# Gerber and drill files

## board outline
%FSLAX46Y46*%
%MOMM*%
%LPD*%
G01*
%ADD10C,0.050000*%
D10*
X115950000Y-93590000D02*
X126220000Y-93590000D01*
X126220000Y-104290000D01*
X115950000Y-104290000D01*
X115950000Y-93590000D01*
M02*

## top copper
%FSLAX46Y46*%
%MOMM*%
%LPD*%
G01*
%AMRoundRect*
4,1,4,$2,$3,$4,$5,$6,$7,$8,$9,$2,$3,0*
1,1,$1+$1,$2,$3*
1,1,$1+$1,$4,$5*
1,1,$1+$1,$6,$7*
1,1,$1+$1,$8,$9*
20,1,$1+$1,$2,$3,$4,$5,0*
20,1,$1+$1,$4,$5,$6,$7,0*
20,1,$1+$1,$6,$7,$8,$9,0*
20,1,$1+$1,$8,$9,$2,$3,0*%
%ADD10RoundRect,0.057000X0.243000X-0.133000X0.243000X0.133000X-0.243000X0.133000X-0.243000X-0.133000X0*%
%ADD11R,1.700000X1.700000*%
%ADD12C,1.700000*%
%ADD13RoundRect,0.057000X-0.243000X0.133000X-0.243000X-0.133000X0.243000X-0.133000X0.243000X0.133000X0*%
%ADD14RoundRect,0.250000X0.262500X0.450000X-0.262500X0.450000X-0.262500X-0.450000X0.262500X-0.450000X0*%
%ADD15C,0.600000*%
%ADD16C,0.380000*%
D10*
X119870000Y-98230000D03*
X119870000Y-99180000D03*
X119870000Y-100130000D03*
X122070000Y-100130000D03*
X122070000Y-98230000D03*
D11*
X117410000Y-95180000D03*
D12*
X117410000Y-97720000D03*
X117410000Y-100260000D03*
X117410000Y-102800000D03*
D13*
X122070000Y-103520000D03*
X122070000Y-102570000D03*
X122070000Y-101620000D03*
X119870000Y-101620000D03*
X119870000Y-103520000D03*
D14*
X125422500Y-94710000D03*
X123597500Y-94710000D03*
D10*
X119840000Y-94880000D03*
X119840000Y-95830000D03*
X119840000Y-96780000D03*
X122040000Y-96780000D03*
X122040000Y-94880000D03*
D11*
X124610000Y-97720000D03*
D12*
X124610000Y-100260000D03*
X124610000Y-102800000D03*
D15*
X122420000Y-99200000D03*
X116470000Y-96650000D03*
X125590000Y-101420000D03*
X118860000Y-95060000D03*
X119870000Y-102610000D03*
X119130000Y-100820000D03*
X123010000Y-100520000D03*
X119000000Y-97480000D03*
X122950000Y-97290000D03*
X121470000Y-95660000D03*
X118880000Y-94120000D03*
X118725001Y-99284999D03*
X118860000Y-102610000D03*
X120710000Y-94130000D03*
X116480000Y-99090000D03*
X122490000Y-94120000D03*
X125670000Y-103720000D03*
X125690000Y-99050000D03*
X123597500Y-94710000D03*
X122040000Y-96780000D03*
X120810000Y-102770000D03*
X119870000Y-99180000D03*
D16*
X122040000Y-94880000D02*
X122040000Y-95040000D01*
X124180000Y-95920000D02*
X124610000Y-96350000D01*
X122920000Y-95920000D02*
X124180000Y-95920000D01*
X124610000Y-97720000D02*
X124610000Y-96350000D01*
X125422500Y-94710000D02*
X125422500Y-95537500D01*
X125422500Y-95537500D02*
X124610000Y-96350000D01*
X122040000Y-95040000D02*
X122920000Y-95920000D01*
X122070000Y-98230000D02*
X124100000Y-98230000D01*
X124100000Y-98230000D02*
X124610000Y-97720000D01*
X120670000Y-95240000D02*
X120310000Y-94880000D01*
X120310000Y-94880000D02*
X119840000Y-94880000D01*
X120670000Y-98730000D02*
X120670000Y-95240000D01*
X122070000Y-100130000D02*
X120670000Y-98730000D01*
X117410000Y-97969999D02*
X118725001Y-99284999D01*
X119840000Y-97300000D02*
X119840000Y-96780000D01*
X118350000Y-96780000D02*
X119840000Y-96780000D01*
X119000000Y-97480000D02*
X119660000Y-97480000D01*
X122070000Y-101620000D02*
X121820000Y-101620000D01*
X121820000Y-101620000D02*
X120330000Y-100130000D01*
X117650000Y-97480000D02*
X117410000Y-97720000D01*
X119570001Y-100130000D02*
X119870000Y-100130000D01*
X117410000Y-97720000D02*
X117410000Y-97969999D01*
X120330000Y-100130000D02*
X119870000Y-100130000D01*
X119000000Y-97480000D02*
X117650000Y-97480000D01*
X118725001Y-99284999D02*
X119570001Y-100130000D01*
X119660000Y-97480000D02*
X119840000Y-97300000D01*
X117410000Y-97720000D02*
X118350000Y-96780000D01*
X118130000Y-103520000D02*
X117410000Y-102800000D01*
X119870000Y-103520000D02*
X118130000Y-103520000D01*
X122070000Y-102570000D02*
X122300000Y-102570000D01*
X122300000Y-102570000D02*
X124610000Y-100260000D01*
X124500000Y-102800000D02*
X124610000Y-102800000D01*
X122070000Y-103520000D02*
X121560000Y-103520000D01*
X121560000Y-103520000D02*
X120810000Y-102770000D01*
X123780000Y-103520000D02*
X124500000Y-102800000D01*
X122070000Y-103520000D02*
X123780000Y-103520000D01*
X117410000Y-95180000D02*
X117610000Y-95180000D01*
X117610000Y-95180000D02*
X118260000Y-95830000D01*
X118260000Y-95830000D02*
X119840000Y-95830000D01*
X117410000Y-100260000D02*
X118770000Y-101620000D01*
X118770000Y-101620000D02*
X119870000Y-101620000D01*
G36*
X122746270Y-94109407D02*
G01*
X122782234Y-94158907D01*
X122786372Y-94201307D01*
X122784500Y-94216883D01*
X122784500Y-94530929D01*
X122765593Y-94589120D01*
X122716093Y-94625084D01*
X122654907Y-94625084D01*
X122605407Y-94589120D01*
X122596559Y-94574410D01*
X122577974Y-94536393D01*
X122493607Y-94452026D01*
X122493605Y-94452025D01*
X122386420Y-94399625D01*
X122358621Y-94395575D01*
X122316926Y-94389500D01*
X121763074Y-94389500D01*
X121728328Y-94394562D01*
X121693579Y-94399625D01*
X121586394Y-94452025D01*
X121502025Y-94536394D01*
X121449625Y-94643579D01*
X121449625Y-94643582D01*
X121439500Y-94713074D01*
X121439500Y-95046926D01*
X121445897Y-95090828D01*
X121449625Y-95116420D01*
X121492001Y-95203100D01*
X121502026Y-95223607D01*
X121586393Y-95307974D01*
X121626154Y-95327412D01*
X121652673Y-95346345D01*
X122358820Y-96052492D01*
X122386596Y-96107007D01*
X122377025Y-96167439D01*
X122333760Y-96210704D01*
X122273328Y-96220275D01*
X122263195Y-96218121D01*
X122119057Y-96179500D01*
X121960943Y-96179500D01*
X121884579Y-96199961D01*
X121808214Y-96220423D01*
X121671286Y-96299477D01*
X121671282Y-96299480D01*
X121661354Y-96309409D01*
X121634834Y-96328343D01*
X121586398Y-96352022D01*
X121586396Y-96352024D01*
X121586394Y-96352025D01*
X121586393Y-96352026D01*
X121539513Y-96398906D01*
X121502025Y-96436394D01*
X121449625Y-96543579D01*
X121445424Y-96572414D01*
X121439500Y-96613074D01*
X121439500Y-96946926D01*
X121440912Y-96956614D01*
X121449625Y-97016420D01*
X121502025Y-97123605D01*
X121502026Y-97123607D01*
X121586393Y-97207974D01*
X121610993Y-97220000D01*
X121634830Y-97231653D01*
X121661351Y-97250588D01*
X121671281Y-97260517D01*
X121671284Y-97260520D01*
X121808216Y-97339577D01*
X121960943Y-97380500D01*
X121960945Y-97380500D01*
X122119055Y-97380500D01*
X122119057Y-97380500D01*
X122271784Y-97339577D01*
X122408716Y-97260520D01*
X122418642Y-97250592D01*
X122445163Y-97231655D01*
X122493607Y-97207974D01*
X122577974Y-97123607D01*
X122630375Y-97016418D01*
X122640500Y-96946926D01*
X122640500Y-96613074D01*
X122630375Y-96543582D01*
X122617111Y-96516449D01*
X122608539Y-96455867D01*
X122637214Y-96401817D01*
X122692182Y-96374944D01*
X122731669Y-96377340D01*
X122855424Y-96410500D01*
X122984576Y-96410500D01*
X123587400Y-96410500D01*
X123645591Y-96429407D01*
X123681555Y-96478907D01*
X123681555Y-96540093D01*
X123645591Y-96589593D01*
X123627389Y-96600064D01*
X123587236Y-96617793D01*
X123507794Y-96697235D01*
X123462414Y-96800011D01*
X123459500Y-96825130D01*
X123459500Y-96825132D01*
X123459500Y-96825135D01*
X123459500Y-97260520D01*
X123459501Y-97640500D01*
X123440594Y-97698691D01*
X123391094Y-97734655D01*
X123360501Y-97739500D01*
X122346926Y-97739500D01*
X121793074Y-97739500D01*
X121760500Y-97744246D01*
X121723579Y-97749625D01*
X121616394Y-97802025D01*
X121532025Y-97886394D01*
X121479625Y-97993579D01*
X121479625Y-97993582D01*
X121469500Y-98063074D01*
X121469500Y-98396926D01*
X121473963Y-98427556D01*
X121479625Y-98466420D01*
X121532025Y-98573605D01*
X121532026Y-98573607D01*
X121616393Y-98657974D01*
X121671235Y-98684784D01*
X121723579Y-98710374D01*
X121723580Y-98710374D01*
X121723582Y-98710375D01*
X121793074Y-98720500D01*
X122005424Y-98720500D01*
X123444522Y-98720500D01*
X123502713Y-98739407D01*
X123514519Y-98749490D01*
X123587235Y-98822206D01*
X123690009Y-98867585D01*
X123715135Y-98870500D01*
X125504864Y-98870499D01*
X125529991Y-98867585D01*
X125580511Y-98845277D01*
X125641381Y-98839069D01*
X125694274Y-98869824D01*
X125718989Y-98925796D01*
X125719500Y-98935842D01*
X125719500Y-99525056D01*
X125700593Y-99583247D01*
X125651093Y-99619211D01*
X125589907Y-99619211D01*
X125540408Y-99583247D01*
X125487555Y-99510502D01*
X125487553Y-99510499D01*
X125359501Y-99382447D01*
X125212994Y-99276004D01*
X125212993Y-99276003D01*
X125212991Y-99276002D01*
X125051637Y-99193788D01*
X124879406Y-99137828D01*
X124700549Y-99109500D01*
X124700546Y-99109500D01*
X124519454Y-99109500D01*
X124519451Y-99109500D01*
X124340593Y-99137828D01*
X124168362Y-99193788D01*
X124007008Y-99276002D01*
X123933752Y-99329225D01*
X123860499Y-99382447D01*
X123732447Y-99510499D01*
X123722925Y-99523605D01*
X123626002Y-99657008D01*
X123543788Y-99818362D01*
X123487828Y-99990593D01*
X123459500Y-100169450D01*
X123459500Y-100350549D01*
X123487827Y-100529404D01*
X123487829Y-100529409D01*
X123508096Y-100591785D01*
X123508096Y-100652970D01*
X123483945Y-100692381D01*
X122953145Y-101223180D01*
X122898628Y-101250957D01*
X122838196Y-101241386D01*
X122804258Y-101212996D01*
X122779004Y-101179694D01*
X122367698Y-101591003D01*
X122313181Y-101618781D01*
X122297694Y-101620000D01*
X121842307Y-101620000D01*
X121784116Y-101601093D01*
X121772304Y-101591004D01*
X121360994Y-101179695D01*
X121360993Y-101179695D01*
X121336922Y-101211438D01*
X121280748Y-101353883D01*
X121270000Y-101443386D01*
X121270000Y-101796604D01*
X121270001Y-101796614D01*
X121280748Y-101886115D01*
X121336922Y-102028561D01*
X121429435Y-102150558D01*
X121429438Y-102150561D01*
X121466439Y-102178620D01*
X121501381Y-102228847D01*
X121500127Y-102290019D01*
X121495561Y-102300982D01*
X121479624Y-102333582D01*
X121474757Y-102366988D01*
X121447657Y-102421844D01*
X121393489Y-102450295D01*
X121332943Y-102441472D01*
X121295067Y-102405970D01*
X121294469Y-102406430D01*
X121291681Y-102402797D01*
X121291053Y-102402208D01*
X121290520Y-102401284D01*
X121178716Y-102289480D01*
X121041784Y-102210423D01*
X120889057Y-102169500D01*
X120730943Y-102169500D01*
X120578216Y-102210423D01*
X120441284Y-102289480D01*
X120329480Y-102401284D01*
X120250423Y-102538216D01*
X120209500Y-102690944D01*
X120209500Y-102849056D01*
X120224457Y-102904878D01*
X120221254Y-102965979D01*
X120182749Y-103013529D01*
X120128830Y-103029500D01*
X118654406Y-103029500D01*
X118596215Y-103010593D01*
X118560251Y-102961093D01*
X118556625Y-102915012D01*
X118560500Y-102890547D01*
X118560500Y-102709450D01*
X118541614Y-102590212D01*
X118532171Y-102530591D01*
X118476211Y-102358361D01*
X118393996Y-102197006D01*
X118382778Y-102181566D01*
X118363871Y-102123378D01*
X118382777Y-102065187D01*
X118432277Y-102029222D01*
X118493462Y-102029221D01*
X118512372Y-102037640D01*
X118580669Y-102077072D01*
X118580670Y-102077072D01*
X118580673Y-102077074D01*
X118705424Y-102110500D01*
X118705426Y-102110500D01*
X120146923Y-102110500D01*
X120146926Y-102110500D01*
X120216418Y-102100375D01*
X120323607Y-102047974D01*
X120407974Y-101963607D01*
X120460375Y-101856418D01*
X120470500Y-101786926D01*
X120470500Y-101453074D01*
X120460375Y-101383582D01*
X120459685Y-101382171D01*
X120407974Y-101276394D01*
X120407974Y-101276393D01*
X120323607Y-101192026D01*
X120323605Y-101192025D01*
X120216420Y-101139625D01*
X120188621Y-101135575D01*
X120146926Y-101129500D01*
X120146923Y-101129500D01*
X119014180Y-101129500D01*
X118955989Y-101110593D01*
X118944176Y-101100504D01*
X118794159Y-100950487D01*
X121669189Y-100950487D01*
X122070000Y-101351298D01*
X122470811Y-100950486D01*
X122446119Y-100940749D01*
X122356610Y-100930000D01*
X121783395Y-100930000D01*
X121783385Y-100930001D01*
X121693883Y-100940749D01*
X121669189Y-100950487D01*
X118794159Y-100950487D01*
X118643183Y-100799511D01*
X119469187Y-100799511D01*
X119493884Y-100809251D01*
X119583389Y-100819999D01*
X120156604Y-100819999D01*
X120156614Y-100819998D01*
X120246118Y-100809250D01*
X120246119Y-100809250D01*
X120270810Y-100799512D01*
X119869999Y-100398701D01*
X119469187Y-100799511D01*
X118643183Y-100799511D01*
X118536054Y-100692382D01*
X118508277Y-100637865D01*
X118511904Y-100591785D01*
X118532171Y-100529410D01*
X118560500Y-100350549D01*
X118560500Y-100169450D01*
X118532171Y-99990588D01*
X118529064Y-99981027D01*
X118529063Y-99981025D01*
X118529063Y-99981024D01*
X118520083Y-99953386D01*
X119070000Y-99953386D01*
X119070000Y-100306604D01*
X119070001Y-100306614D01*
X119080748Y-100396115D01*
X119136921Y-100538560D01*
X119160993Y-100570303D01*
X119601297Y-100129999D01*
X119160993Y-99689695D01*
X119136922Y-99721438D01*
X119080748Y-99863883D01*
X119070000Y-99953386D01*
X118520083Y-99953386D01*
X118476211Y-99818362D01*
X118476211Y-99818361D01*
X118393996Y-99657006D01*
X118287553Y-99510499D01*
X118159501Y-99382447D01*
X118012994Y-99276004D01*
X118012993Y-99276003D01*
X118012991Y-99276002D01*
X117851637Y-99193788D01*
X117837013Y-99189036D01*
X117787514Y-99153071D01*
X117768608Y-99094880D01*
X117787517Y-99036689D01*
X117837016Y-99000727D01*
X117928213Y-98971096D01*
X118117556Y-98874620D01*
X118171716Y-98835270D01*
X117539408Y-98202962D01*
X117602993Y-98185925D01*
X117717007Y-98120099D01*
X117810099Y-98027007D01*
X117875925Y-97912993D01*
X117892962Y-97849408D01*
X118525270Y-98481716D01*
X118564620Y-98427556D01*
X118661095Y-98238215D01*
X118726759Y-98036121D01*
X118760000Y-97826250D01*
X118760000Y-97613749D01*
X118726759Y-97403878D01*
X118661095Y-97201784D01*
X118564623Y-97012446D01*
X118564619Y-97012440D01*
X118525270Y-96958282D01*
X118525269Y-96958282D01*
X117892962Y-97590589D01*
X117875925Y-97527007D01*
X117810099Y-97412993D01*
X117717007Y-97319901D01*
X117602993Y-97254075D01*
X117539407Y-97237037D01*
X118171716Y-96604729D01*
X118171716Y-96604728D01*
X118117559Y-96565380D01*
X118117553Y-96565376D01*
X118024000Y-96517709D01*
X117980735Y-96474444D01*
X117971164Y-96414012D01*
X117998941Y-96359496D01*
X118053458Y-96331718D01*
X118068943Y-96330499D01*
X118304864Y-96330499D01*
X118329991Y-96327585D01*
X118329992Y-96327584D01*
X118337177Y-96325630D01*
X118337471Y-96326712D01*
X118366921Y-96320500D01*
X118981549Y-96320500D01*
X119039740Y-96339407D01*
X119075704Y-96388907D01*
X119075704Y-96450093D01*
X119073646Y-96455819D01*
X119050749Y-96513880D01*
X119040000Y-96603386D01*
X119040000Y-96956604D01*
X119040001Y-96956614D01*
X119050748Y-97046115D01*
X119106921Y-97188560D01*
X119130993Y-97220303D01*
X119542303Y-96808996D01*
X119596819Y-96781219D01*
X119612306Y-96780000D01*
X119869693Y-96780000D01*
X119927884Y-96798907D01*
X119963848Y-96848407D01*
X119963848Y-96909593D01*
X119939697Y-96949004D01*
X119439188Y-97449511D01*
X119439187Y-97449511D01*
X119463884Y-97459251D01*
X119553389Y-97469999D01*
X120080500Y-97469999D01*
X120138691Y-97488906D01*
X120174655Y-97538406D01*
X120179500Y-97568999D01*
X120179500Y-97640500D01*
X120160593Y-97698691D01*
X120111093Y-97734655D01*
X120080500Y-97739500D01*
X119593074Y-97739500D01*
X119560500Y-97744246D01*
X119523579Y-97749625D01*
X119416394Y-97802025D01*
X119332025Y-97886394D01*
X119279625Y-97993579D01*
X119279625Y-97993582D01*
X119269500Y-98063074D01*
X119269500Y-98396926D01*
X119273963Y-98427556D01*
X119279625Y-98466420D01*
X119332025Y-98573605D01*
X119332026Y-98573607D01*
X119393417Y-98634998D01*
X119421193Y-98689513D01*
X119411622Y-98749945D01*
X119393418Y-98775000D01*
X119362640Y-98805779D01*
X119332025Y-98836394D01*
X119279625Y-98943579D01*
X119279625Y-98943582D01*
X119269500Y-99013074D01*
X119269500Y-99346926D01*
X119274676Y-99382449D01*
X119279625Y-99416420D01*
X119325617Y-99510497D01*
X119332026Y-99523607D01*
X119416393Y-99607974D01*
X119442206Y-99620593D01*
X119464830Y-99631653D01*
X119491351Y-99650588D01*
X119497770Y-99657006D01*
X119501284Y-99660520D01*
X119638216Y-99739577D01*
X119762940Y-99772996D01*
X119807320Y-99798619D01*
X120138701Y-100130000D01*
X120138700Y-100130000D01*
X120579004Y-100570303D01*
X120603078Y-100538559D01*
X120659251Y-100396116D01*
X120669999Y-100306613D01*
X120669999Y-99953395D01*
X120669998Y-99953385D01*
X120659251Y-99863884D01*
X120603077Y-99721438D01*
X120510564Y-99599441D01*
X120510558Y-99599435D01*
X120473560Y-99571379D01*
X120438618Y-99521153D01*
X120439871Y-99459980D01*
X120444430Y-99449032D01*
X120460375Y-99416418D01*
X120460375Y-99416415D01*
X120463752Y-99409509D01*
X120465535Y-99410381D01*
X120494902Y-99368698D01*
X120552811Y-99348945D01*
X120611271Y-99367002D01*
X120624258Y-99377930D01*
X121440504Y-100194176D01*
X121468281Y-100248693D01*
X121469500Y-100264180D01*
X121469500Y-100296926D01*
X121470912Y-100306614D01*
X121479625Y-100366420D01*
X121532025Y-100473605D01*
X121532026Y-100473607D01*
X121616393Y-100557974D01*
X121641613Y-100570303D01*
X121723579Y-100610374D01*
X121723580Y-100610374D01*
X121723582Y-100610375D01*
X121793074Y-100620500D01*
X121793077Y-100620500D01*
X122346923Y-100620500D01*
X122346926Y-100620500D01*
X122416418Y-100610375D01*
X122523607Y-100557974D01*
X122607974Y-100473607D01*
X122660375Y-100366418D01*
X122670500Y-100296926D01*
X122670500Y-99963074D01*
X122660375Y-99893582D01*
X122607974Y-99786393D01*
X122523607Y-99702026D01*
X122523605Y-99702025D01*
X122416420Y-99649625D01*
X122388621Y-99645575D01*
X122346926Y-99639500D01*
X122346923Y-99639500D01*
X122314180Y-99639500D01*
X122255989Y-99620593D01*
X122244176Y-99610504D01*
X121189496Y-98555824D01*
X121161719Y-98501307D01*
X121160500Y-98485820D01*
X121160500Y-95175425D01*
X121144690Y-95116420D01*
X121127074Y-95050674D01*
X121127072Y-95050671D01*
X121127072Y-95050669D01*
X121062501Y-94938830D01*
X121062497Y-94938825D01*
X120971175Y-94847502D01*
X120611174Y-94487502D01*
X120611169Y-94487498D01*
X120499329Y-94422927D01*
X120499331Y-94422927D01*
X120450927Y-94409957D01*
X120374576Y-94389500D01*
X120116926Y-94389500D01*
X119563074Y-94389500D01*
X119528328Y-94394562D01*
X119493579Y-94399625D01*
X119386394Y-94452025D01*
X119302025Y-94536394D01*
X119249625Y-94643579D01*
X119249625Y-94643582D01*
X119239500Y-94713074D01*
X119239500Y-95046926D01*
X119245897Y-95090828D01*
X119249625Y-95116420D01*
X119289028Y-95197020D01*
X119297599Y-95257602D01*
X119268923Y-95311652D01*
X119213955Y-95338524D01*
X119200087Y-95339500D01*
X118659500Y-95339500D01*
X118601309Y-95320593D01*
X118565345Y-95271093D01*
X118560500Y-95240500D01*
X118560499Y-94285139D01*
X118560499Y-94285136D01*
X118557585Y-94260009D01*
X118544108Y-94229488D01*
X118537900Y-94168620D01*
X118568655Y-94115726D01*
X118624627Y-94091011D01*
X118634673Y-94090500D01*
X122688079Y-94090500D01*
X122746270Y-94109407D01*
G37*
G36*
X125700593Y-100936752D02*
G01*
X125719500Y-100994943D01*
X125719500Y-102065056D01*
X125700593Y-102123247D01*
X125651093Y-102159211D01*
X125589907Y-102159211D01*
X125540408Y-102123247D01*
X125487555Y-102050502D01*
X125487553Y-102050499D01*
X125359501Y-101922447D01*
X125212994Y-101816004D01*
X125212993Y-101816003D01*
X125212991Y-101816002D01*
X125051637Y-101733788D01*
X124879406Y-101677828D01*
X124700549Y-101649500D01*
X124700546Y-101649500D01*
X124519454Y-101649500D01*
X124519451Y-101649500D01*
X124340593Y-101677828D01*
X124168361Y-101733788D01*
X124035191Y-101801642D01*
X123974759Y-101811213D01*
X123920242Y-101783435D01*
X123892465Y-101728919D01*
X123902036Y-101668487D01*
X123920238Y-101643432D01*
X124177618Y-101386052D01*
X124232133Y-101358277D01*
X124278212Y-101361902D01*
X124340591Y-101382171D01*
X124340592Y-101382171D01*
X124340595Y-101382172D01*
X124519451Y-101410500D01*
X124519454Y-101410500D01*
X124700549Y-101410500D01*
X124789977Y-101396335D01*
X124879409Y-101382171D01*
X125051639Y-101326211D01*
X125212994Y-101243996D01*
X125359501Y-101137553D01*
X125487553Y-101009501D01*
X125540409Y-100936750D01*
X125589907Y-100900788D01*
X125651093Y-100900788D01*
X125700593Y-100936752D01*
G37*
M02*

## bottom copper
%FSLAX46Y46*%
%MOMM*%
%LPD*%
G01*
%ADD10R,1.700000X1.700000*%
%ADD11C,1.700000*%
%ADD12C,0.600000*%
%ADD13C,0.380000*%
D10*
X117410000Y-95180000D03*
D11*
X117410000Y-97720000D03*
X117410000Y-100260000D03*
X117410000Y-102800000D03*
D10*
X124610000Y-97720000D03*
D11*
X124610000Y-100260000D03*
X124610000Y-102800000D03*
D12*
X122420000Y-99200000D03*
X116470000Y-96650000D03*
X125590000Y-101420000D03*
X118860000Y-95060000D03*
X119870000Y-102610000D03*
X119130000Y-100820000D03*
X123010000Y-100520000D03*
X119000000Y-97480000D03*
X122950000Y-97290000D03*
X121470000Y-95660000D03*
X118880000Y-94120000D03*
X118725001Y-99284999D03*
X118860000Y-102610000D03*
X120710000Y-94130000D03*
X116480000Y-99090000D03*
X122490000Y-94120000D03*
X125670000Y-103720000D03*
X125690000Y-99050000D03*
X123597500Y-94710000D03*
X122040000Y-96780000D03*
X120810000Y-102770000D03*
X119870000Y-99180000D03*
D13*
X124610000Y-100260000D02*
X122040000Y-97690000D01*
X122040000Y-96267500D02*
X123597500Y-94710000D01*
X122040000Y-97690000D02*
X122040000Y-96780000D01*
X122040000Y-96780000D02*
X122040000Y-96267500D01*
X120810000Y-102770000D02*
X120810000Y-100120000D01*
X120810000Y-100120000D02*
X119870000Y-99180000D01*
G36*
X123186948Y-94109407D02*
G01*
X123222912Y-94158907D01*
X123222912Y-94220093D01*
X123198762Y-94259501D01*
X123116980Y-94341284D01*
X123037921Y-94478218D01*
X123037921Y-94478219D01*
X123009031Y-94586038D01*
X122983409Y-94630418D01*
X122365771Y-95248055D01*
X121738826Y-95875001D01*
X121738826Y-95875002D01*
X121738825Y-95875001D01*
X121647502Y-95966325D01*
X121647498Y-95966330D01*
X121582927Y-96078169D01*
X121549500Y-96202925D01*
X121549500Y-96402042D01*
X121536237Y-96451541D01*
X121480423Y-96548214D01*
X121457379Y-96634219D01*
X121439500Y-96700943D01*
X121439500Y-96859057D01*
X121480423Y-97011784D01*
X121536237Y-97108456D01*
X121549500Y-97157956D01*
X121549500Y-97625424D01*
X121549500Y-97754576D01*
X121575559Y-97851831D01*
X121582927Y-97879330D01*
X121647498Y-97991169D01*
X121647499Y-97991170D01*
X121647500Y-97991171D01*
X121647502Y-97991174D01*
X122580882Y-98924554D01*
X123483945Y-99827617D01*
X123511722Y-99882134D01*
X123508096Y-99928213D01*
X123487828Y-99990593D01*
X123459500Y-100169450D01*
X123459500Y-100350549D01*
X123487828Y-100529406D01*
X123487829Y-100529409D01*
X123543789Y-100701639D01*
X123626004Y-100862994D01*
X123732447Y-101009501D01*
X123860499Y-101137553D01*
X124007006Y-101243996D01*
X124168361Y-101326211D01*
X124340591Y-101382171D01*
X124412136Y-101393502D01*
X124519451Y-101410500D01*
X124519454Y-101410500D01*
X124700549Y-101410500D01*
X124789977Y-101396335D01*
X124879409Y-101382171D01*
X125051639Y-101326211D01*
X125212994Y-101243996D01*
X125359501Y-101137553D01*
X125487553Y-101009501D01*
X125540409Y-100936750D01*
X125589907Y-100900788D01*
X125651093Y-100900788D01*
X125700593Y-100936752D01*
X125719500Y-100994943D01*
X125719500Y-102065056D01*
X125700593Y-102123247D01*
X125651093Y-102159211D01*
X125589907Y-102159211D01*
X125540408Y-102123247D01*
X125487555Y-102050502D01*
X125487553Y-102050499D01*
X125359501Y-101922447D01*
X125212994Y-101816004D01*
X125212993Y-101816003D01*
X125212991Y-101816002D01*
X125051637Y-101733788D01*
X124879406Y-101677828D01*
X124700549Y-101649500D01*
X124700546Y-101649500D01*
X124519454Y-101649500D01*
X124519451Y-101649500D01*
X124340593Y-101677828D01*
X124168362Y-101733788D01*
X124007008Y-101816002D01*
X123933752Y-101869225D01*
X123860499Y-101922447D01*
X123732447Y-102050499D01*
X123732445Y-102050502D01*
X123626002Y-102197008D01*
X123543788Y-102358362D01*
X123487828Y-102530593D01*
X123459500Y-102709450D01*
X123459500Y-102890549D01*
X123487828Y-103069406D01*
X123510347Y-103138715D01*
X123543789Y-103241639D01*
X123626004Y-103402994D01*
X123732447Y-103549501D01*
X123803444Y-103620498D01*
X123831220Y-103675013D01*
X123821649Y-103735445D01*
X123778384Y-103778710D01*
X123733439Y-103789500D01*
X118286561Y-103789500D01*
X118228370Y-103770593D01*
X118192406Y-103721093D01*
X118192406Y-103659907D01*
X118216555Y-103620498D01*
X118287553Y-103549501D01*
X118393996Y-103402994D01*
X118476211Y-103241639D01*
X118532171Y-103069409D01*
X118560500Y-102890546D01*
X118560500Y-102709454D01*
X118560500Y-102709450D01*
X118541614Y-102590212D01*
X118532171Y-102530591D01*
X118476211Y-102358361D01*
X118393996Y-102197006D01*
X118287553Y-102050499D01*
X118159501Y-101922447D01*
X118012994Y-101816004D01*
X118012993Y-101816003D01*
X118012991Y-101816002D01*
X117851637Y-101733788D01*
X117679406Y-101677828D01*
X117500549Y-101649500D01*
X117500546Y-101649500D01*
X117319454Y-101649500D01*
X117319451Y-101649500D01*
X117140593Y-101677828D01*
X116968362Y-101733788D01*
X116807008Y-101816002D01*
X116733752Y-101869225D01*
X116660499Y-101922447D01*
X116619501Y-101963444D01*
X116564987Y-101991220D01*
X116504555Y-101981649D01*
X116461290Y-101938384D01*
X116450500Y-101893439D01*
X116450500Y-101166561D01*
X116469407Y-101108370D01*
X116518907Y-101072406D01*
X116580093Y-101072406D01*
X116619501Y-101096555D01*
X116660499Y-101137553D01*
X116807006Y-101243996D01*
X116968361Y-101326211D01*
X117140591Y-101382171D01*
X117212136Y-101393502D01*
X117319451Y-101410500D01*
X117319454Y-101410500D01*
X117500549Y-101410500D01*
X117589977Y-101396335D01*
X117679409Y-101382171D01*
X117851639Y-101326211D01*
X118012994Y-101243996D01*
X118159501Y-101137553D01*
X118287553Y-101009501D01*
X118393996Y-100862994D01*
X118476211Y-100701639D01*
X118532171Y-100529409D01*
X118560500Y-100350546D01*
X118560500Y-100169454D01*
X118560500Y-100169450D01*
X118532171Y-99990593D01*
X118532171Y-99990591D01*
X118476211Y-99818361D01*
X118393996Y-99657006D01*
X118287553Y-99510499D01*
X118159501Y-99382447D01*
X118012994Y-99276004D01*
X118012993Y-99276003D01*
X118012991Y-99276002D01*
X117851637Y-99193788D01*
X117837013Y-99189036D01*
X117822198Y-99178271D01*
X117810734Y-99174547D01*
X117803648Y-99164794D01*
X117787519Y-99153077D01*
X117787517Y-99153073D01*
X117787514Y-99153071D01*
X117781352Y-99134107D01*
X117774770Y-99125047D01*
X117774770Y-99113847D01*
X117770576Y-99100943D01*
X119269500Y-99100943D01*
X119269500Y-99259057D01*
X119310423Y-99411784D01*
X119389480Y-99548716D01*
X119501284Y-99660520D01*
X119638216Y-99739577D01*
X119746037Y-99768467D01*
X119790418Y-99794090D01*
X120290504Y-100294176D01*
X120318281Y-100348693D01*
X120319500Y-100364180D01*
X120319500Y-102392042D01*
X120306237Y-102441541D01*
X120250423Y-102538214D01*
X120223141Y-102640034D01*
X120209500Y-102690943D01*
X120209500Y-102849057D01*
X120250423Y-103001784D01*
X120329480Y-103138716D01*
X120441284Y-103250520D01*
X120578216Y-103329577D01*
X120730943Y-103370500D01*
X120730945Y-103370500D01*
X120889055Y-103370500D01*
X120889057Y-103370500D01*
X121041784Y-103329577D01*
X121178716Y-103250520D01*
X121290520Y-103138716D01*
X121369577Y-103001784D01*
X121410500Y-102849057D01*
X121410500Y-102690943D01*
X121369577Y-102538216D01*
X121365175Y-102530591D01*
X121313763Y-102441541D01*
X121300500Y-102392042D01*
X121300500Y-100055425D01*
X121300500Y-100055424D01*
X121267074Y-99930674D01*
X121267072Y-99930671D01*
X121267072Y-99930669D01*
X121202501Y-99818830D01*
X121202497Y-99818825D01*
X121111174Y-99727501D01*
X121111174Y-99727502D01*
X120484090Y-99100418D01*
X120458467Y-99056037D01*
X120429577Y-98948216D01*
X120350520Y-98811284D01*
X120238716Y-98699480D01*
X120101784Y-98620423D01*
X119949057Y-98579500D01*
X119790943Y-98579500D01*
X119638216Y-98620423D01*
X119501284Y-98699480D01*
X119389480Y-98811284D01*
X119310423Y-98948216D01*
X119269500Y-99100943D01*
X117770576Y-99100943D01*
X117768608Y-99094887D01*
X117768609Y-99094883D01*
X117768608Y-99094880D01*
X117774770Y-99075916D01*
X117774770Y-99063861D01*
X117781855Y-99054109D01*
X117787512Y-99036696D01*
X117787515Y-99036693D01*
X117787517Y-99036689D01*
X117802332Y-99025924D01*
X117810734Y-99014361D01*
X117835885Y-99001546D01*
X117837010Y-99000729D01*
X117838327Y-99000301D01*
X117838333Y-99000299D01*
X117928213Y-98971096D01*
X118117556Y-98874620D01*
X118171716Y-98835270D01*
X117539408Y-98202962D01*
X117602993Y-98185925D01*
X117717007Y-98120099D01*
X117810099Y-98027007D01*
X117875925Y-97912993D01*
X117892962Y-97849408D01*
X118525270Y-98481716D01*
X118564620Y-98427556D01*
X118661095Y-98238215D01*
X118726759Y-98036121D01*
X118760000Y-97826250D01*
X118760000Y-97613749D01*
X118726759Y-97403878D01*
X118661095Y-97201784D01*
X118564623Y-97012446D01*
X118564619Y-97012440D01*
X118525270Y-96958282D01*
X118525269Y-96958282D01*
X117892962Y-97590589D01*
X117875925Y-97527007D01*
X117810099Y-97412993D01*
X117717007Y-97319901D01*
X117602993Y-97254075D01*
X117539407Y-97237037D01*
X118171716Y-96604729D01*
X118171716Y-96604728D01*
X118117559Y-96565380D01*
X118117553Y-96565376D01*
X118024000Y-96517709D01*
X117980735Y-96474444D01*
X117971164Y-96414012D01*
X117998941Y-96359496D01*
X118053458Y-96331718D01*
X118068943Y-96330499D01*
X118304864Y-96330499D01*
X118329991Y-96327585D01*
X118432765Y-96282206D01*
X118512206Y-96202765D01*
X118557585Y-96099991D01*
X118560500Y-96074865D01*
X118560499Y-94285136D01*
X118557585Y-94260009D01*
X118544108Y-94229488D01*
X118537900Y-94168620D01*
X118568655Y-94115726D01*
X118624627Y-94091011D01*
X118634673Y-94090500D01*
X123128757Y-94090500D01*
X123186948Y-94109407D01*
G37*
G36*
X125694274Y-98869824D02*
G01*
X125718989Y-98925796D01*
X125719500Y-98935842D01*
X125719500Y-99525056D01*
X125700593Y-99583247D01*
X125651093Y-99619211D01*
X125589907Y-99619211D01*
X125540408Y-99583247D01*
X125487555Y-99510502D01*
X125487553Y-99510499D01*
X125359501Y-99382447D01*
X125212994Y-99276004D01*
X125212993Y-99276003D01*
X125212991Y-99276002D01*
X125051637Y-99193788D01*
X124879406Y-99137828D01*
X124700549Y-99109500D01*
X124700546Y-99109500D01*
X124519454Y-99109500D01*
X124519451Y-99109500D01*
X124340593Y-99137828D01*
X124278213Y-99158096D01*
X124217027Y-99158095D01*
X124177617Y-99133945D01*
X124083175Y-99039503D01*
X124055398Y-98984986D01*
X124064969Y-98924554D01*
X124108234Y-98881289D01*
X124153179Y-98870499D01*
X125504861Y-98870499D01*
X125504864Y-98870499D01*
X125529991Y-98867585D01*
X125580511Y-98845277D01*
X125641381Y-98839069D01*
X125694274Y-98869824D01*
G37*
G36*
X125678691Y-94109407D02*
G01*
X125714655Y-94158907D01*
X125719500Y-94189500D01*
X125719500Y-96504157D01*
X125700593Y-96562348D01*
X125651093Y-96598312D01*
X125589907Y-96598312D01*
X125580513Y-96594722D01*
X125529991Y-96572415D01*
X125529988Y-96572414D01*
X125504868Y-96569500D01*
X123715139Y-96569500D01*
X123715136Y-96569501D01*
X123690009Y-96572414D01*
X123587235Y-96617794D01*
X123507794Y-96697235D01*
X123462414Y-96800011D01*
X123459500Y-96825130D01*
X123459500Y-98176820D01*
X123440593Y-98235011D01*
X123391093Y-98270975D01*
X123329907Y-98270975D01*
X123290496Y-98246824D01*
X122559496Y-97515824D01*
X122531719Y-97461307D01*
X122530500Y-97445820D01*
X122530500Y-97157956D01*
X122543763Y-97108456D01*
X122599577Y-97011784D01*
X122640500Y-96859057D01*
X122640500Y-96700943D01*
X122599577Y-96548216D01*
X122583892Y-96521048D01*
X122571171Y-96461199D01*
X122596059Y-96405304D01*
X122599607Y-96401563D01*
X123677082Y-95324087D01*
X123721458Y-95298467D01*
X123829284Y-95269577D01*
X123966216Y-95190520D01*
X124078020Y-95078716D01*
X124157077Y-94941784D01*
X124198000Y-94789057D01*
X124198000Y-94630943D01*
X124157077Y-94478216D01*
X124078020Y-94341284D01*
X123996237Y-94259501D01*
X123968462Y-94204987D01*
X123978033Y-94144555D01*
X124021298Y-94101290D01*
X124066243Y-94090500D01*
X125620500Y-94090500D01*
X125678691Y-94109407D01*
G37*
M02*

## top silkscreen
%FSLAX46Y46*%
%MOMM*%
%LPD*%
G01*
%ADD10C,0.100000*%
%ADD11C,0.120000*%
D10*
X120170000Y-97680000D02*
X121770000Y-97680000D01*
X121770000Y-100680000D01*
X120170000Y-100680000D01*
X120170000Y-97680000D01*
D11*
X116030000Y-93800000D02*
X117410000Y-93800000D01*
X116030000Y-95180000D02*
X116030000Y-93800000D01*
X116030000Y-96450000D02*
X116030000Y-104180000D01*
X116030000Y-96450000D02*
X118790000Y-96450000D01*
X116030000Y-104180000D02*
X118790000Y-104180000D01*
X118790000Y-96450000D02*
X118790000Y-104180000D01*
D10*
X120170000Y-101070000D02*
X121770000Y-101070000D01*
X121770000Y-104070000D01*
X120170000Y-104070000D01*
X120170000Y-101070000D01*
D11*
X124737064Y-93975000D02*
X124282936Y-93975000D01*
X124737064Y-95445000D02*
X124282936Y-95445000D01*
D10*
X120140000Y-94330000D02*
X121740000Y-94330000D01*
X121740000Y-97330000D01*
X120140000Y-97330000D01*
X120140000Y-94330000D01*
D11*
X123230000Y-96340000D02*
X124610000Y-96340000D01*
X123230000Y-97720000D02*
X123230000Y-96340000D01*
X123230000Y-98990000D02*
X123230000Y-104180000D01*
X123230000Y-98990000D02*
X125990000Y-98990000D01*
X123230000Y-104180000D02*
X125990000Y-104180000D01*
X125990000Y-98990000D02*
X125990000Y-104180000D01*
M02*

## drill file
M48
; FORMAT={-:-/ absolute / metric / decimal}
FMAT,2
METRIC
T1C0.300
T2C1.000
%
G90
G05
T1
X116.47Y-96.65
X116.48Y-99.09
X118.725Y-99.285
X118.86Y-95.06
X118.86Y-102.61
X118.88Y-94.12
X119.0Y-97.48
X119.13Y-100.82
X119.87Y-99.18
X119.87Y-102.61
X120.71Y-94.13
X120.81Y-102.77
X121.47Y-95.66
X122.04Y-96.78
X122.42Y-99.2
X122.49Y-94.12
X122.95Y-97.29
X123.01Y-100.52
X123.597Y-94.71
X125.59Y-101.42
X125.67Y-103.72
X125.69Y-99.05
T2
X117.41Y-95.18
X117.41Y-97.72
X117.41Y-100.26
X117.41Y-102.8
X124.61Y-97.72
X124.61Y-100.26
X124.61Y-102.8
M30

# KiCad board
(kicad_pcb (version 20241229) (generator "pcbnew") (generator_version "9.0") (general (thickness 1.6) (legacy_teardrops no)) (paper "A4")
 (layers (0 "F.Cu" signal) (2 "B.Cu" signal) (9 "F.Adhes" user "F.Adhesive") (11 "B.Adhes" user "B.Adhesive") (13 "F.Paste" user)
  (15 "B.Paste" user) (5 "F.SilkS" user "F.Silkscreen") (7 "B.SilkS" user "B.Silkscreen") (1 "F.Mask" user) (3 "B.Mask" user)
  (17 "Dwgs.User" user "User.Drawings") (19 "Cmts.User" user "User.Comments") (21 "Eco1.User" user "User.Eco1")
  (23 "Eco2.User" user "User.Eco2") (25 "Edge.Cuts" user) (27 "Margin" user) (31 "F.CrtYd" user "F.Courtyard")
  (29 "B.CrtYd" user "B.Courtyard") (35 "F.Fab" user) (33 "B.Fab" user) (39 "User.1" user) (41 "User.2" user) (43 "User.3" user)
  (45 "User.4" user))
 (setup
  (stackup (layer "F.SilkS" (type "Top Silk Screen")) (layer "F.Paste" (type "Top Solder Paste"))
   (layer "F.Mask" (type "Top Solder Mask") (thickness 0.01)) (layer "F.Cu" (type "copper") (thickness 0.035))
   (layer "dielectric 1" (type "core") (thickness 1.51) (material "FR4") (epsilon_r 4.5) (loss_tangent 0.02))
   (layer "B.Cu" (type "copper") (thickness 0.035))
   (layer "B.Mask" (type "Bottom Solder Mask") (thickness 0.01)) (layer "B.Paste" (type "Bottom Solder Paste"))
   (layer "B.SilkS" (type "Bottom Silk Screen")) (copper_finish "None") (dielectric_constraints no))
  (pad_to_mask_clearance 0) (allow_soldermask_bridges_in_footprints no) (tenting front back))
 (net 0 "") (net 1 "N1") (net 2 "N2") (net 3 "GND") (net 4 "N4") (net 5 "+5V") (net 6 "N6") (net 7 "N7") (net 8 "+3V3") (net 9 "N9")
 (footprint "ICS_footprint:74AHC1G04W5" (layer "F.Cu") (at 120.97 99.18 90)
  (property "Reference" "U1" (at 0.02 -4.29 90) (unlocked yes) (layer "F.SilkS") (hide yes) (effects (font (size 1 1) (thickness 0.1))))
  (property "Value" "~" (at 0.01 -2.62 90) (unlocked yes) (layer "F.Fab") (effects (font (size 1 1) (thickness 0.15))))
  (fp_rect (start -1.5 -0.8) (end 1.5 0.8) (stroke (width 0.1) (type solid)) (fill no) (layer "F.SilkS"))
  (pad "1" smd roundrect (at 0.95 -1.1 90) (size 0.38 0.6) (layers "F.Cu" "F.Mask" "F.Paste") (roundrect_rratio 0.15) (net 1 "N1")
   (thermal_bridge_angle 45))
  (pad "2" smd roundrect (at 0 -1.1 90) (size 0.38 0.6) (layers "F.Cu" "F.Mask" "F.Paste") (roundrect_rratio 0.15) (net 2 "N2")
   (thermal_bridge_angle 45))
  (pad "3" smd roundrect (at -0.95 -1.1 90) (size 0.38 0.6) (layers "F.Cu" "F.Mask" "F.Paste") (roundrect_rratio 0.15) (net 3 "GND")
   (thermal_bridge_angle 45))
  (pad "4" smd roundrect (at -0.95 1.1 90) (size 0.38 0.6) (layers "F.Cu" "F.Mask" "F.Paste") (roundrect_rratio 0.15) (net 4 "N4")
   (thermal_bridge_angle 45))
  (pad "5" smd roundrect (at 0.95 1.1 90) (size 0.38 0.6) (layers "F.Cu" "F.Mask" "F.Paste") (roundrect_rratio 0.15) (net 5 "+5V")
   (thermal_bridge_angle 45)))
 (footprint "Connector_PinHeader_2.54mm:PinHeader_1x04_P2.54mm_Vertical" (layer "F.Cu") (at 117.41 95.18)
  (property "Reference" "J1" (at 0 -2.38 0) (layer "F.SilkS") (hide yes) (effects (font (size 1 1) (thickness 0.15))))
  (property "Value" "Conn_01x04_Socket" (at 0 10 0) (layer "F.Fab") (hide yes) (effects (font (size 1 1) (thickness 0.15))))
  (fp_line (start -1.38 -1.38) (end 0 -1.38) (stroke (width 0.12) (type solid)) (layer "F.SilkS"))
  (fp_line (start -1.38 0) (end -1.38 -1.38) (stroke (width 0.12) (type solid)) (layer "F.SilkS"))
  (fp_line (start -1.38 1.27) (end -1.38 9) (stroke (width 0.12) (type solid)) (layer "F.SilkS"))
  (fp_line (start -1.38 1.27) (end 1.38 1.27) (stroke (width 0.12) (type solid)) (layer "F.SilkS"))
  (fp_line (start -1.38 9) (end 1.38 9) (stroke (width 0.12) (type solid)) (layer "F.SilkS"))
  (fp_line (start 1.38 1.27) (end 1.38 9) (stroke (width 0.12) (type solid)) (layer "F.SilkS"))
  (pad "1" thru_hole rect (at 0 0) (size 1.7 1.7) (drill 1) (layers "*.Cu" "*.Mask") (remove_unused_layers no) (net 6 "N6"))
  (pad "2" thru_hole circle (at 0 2.54) (size 1.7 1.7) (drill 1) (layers "*.Cu" "*.Mask") (remove_unused_layers no) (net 3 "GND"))
  (pad "3" thru_hole circle (at 0 5.08) (size 1.7 1.7) (drill 1) (layers "*.Cu" "*.Mask") (remove_unused_layers no) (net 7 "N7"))
  (pad "4" thru_hole circle (at 0 7.62) (size 1.7 1.7) (drill 1) (layers "*.Cu" "*.Mask") (remove_unused_layers no) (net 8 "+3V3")))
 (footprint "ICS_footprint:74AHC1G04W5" (layer "F.Cu") (at 120.97 102.57 -90)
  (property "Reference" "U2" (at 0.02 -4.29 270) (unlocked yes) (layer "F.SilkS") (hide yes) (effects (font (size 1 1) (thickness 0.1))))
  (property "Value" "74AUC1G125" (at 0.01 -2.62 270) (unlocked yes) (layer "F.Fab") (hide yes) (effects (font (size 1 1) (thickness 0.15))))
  (fp_rect (start -1.5 -0.8) (end 1.5 0.8) (stroke (width 0.1) (type solid)) (fill no) (layer "F.SilkS"))
  (pad "1" smd roundrect (at 0.95 -1.1 270) (size 0.38 0.6) (layers "F.Cu" "F.Mask" "F.Paste") (roundrect_rratio 0.15) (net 2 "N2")
   (thermal_bridge_angle 45))
  (pad "2" smd roundrect (at 0 -1.1 270) (size 0.38 0.6) (layers "F.Cu" "F.Mask" "F.Paste") (roundrect_rratio 0.15) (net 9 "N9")
   (thermal_bridge_angle 45))
  (pad "3" smd roundrect (at -0.95 -1.1 270) (size 0.38 0.6) (layers "F.Cu" "F.Mask" "F.Paste") (roundrect_rratio 0.15) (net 3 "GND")
   (thermal_bridge_angle 45))
  (pad "4" smd roundrect (at -0.95 1.1 270) (size 0.38 0.6) (layers "F.Cu" "F.Mask" "F.Paste") (roundrect_rratio 0.15) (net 7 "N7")
   (thermal_bridge_angle 45))
  (pad "5" smd roundrect (at 0.95 1.1 270) (size 0.38 0.6) (layers "F.Cu" "F.Mask" "F.Paste") (roundrect_rratio 0.15) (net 8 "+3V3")
   (thermal_bridge_angle 45)))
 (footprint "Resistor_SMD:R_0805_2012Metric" (layer "F.Cu") (at 124.51 94.71 180)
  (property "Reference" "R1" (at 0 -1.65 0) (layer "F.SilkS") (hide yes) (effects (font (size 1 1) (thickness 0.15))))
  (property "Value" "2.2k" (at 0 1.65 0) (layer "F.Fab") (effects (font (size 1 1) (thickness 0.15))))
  (fp_line (start -0.227064 0.735) (end 0.227064 0.735) (stroke (width 0.12) (type solid)) (layer "F.SilkS"))
  (fp_line (start -0.227064 -0.735) (end 0.227064 -0.735) (stroke (width 0.12) (type solid)) (layer "F.SilkS"))
  (pad "1" smd roundrect (at -0.9125 0 180) (size 1.025 1.4) (layers "F.Cu" "F.Mask" "F.Paste") (roundrect_rratio 0.243902) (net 5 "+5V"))
  (pad "2" smd roundrect (at 0.9125 0 180) (size 1.025 1.4) (layers "F.Cu" "F.Mask" "F.Paste") (roundrect_rratio 0.243902) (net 9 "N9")))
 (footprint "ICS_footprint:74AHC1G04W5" (layer "F.Cu") (at 120.94 95.83 90)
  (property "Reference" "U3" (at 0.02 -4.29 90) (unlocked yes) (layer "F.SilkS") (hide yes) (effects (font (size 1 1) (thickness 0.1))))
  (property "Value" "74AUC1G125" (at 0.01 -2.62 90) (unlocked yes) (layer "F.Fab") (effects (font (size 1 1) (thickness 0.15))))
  (fp_rect (start -1.5 -0.8) (end 1.5 0.8) (stroke (width 0.1) (type solid)) (fill no) (layer "F.SilkS"))
  (pad "1" smd roundrect (at 0.95 -1.1 90) (size 0.38 0.6) (layers "F.Cu" "F.Mask" "F.Paste") (roundrect_rratio 0.15) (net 4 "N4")
   (thermal_bridge_angle 45))
  (pad "2" smd roundrect (at 0 -1.1 90) (size 0.38 0.6) (layers "F.Cu" "F.Mask" "F.Paste") (roundrect_rratio 0.15) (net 6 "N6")
   (thermal_bridge_angle 45))
  (pad "3" smd roundrect (at -0.95 -1.1 90) (size 0.38 0.6) (layers "F.Cu" "F.Mask" "F.Paste") (roundrect_rratio 0.15) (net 3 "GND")
   (thermal_bridge_angle 45))
  (pad "4" smd roundrect (at -0.95 1.1 90) (size 0.38 0.6) (layers "F.Cu" "F.Mask" "F.Paste") (roundrect_rratio 0.15) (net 9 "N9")
   (thermal_bridge_angle 45))
  (pad "5" smd roundrect (at 0.95 1.1 90) (size 0.38 0.6) (layers "F.Cu" "F.Mask" "F.Paste") (roundrect_rratio 0.15) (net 5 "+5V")
   (thermal_bridge_angle 45)))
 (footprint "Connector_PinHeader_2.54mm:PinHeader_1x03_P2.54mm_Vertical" (layer "F.Cu") (at 124.61 97.72)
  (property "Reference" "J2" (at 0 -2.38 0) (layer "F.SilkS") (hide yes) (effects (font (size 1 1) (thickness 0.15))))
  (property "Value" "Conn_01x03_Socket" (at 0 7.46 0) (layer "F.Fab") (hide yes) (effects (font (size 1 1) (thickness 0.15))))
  (fp_line (start -1.38 -1.38) (end 0 -1.38) (stroke (width 0.12) (type solid)) (layer "F.SilkS"))
  (fp_line (start -1.38 0) (end -1.38 -1.38) (stroke (width 0.12) (type solid)) (layer "F.SilkS"))
  (fp_line (start -1.38 1.27) (end -1.38 6.46) (stroke (width 0.12) (type solid)) (layer "F.SilkS"))
  (fp_line (start -1.38 1.27) (end 1.38 1.27) (stroke (width 0.12) (type solid)) (layer "F.SilkS"))
  (fp_line (start -1.38 6.46) (end 1.38 6.46) (stroke (width 0.12) (type solid)) (layer "F.SilkS"))
  (fp_line (start 1.38 1.27) (end 1.38 6.46) (stroke (width 0.12) (type solid)) (layer "F.SilkS"))
  (pad "1" thru_hole rect (at 0 0) (size 1.7 1.7) (drill 1) (layers "*.Cu" "*.Mask") (remove_unused_layers no) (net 5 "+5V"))
  (pad "2" thru_hole circle (at 0 2.54) (size 1.7 1.7) (drill 1) (layers "*.Cu" "*.Mask") (remove_unused_layers no) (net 9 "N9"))
  (pad "3" thru_hole circle (at 0 5.08) (size 1.7 1.7) (drill 1) (layers "*.Cu" "*.Mask") (remove_unused_layers no) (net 2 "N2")))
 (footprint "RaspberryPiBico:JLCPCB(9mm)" (layer "B.Cu") (at 121.22467 98.45426 115)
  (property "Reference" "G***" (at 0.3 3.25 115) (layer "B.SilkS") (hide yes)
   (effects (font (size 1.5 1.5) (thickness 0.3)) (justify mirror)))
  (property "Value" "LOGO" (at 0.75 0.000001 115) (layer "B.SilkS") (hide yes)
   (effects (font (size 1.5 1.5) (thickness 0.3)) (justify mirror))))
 (gr_rect (start 115.95 93.59) (end 126.22 104.29) (stroke (width 0.05) (type default)) (fill no) (layer "Edge.Cuts"))
 (segment (start 122.04 94.88) (end 122.04 95.04) (width 0.38) (layer "F.Cu") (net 5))
 (segment (start 124.18 95.92) (end 124.61 96.35) (width 0.38) (layer "F.Cu") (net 5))
 (segment (start 122.92 95.92) (end 124.18 95.92) (width 0.38) (layer "F.Cu") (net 5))
 (segment (start 124.61 97.72) (end 124.61 96.35) (width 0.38) (layer "F.Cu") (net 5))
 (segment (start 125.4225 94.71) (end 125.4225 95.5375) (width 0.38) (layer "F.Cu") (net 5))
 (segment (start 125.4225 95.5375) (end 124.61 96.35) (width 0.38) (layer "F.Cu") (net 5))
 (segment (start 122.04 95.04) (end 122.92 95.92) (width 0.38) (layer "F.Cu") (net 5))
 (segment (start 122.07 98.23) (end 124.1 98.23) (width 0.38) (layer "F.Cu") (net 5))
 (segment (start 124.1 98.23) (end 124.61 97.72) (width 0.38) (layer "F.Cu") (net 5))
 (segment (start 120.67 95.24) (end 120.31 94.88) (width 0.38) (layer "F.Cu") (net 4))
 (segment (start 120.31 94.88) (end 119.84 94.88) (width 0.38) (layer "F.Cu") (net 4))
 (segment (start 120.67 98.73) (end 120.67 95.24) (width 0.38) (layer "F.Cu") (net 4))
 (segment (start 122.07 100.13) (end 120.67 98.73) (width 0.38) (layer "F.Cu") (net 4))
 (segment (start 117.41 97.969999) (end 118.725001 99.284999) (width 0.38) (layer "F.Cu") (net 3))
 (segment (start 119.84 97.3) (end 119.84 96.78) (width 0.38) (layer "F.Cu") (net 3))
 (segment (start 118.35 96.78) (end 119.84 96.78) (width 0.38) (layer "F.Cu") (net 3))
 (segment (start 119 97.48) (end 119.66 97.48) (width 0.38) (layer "F.Cu") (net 3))
 (segment (start 122.07 101.62) (end 121.82 101.62) (width 0.38) (layer "F.Cu") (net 3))
 (segment (start 121.82 101.62) (end 120.33 100.13) (width 0.38) (layer "F.Cu") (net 3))
 (segment (start 117.65 97.48) (end 117.41 97.72) (width 0.38) (layer "F.Cu") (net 3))
 (segment (start 119.570001 100.13) (end 119.87 100.13) (width 0.38) (layer "F.Cu") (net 3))
 (segment (start 117.41 97.72) (end 117.41 97.969999) (width 0.38) (layer "F.Cu") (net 3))
 (segment (start 120.33 100.13) (end 119.87 100.13) (width 0.38) (layer "F.Cu") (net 3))
 (segment (start 119 97.48) (end 117.65 97.48) (width 0.38) (layer "F.Cu") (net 3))
 (segment (start 118.725001 99.284999) (end 119.570001 100.13) (width 0.38) (layer "F.Cu") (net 3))
 (segment (start 119.66 97.48) (end 119.84 97.3) (width 0.38) (layer "F.Cu") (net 3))
 (segment (start 117.41 97.72) (end 118.35 96.78) (width 0.38) (layer "F.Cu") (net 3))
 (via (at 122.42 99.2) (size 0.6) (drill 0.3) (layers "F.Cu" "B.Cu") (free yes) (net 3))
 (via (at 116.47 96.65) (size 0.6) (drill 0.3) (layers "F.Cu" "B.Cu") (free yes) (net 3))
 (via (at 125.59 101.42) (size 0.6) (drill 0.3) (layers "F.Cu" "B.Cu") (free yes) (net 3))
 (via (at 118.86 95.06) (size 0.6) (drill 0.3) (layers "F.Cu" "B.Cu") (free yes) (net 3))
 (via (at 119.87 102.61) (size 0.6) (drill 0.3) (layers "F.Cu" "B.Cu") (free yes) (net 3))
 (via (at 119.13 100.82) (size 0.6) (drill 0.3) (layers "F.Cu" "B.Cu") (free yes) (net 3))
 (via (at 123.01 100.52) (size 0.6) (drill 0.3) (layers "F.Cu" "B.Cu") (free yes) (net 3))
 (via (at 119 97.48) (size 0.6) (drill 0.3) (layers "F.Cu" "B.Cu") (free yes) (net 3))
 (via (at 122.95 97.29) (size 0.6) (drill 0.3) (layers "F.Cu" "B.Cu") (free yes) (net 3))
 (via (at 121.47 95.66) (size 0.6) (drill 0.3) (layers "F.Cu" "B.Cu") (free yes) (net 3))
 (via (at 118.88 94.12) (size 0.6) (drill 0.3) (layers "F.Cu" "B.Cu") (free yes) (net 3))
 (via (at 118.725001 99.284999) (size 0.6) (drill 0.3) (layers "F.Cu" "B.Cu") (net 3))
 (via (at 118.86 102.61) (size 0.6) (drill 0.3) (layers "F.Cu" "B.Cu") (free yes) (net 3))
 (via (at 120.71 94.13) (size 0.6) (drill 0.3) (layers "F.Cu" "B.Cu") (free yes) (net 3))
 (via (at 116.48 99.09) (size 0.6) (drill 0.3) (layers "F.Cu" "B.Cu") (free yes) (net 3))
 (via (at 122.49 94.12) (size 0.6) (drill 0.3) (layers "F.Cu" "B.Cu") (free yes) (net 3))
 (via (at 125.67 103.72) (size 0.6) (drill 0.3) (layers "F.Cu" "B.Cu") (free yes) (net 3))
 (via (at 125.69 99.05) (size 0.6) (drill 0.3) (layers "F.Cu" "B.Cu") (free yes) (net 3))
 (segment (start 118.13 103.52) (end 117.41 102.8) (width 0.38) (layer "F.Cu") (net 8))
 (segment (start 119.87 103.52) (end 118.13 103.52) (width 0.38) (layer "F.Cu") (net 8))
 (segment (start 122.07 102.57) (end 122.3 102.57) (width 0.38) (layer "F.Cu") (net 9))
 (segment (start 122.3 102.57) (end 124.61 100.26) (width 0.38) (layer "F.Cu") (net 9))
 (via (at 123.5975 94.71) (size 0.6) (drill 0.3) (layers "F.Cu" "B.Cu") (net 9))
 (via (at 122.04 96.78) (size 0.6) (drill 0.3) (layers "F.Cu" "B.Cu") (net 9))
 (segment (start 124.61 100.26) (end 122.04 97.69) (width 0.38) (layer "B.Cu") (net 9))
 (segment (start 122.04 96.2675) (end 123.5975 94.71) (width 0.38) (layer "B.Cu") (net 9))
 (segment (start 122.04 97.69) (end 122.04 96.78) (width 0.38) (layer "B.Cu") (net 9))
 (segment (start 122.04 96.78) (end 122.04 96.2675) (width 0.38) (layer "B.Cu") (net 9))
 (segment (start 124.5 102.8) (end 124.61 102.8) (width 0.38) (layer "F.Cu") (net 2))
 (segment (start 122.07 103.52) (end 121.56 103.52) (width 0.38) (layer "F.Cu") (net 2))
 (segment (start 121.56 103.52) (end 120.81 102.77) (width 0.38) (layer "F.Cu") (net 2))
 (segment (start 123.78 103.52) (end 124.5 102.8) (width 0.38) (layer "F.Cu") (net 2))
 (segment (start 122.07 103.52) (end 123.78 103.52) (width 0.38) (layer "F.Cu") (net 2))
 (via (at 120.81 102.77) (size 0.6) (drill 0.3) (layers "F.Cu" "B.Cu") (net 2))
 (via (at 119.87 99.18) (size 0.6) (drill 0.3) (layers "F.Cu" "B.Cu") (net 2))
 (segment (start 120.81 102.77) (end 120.81 100.12) (width 0.38) (layer "B.Cu") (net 2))
 (segment (start 120.81 100.12) (end 119.87 99.18) (width 0.38) (layer "B.Cu") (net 2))
 (segment (start 117.41 95.18) (end 117.61 95.18) (width 0.38) (layer "F.Cu") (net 6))
 (segment (start 117.61 95.18) (end 118.26 95.83) (width 0.38) (layer "F.Cu") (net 6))
 (segment (start 118.26 95.83) (end 119.84 95.83) (width 0.38) (layer "F.Cu") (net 6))
 (segment (start 117.41 100.26) (end 118.77 101.62) (width 0.38) (layer "F.Cu") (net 7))
 (segment (start 118.77 101.62) (end 119.87 101.62) (width 0.38) (layer "F.Cu") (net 7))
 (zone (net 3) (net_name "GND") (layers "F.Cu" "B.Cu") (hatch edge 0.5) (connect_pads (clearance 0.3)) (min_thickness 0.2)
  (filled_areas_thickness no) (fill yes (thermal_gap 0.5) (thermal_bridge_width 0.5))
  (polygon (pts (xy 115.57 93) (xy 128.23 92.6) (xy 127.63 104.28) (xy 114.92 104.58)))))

